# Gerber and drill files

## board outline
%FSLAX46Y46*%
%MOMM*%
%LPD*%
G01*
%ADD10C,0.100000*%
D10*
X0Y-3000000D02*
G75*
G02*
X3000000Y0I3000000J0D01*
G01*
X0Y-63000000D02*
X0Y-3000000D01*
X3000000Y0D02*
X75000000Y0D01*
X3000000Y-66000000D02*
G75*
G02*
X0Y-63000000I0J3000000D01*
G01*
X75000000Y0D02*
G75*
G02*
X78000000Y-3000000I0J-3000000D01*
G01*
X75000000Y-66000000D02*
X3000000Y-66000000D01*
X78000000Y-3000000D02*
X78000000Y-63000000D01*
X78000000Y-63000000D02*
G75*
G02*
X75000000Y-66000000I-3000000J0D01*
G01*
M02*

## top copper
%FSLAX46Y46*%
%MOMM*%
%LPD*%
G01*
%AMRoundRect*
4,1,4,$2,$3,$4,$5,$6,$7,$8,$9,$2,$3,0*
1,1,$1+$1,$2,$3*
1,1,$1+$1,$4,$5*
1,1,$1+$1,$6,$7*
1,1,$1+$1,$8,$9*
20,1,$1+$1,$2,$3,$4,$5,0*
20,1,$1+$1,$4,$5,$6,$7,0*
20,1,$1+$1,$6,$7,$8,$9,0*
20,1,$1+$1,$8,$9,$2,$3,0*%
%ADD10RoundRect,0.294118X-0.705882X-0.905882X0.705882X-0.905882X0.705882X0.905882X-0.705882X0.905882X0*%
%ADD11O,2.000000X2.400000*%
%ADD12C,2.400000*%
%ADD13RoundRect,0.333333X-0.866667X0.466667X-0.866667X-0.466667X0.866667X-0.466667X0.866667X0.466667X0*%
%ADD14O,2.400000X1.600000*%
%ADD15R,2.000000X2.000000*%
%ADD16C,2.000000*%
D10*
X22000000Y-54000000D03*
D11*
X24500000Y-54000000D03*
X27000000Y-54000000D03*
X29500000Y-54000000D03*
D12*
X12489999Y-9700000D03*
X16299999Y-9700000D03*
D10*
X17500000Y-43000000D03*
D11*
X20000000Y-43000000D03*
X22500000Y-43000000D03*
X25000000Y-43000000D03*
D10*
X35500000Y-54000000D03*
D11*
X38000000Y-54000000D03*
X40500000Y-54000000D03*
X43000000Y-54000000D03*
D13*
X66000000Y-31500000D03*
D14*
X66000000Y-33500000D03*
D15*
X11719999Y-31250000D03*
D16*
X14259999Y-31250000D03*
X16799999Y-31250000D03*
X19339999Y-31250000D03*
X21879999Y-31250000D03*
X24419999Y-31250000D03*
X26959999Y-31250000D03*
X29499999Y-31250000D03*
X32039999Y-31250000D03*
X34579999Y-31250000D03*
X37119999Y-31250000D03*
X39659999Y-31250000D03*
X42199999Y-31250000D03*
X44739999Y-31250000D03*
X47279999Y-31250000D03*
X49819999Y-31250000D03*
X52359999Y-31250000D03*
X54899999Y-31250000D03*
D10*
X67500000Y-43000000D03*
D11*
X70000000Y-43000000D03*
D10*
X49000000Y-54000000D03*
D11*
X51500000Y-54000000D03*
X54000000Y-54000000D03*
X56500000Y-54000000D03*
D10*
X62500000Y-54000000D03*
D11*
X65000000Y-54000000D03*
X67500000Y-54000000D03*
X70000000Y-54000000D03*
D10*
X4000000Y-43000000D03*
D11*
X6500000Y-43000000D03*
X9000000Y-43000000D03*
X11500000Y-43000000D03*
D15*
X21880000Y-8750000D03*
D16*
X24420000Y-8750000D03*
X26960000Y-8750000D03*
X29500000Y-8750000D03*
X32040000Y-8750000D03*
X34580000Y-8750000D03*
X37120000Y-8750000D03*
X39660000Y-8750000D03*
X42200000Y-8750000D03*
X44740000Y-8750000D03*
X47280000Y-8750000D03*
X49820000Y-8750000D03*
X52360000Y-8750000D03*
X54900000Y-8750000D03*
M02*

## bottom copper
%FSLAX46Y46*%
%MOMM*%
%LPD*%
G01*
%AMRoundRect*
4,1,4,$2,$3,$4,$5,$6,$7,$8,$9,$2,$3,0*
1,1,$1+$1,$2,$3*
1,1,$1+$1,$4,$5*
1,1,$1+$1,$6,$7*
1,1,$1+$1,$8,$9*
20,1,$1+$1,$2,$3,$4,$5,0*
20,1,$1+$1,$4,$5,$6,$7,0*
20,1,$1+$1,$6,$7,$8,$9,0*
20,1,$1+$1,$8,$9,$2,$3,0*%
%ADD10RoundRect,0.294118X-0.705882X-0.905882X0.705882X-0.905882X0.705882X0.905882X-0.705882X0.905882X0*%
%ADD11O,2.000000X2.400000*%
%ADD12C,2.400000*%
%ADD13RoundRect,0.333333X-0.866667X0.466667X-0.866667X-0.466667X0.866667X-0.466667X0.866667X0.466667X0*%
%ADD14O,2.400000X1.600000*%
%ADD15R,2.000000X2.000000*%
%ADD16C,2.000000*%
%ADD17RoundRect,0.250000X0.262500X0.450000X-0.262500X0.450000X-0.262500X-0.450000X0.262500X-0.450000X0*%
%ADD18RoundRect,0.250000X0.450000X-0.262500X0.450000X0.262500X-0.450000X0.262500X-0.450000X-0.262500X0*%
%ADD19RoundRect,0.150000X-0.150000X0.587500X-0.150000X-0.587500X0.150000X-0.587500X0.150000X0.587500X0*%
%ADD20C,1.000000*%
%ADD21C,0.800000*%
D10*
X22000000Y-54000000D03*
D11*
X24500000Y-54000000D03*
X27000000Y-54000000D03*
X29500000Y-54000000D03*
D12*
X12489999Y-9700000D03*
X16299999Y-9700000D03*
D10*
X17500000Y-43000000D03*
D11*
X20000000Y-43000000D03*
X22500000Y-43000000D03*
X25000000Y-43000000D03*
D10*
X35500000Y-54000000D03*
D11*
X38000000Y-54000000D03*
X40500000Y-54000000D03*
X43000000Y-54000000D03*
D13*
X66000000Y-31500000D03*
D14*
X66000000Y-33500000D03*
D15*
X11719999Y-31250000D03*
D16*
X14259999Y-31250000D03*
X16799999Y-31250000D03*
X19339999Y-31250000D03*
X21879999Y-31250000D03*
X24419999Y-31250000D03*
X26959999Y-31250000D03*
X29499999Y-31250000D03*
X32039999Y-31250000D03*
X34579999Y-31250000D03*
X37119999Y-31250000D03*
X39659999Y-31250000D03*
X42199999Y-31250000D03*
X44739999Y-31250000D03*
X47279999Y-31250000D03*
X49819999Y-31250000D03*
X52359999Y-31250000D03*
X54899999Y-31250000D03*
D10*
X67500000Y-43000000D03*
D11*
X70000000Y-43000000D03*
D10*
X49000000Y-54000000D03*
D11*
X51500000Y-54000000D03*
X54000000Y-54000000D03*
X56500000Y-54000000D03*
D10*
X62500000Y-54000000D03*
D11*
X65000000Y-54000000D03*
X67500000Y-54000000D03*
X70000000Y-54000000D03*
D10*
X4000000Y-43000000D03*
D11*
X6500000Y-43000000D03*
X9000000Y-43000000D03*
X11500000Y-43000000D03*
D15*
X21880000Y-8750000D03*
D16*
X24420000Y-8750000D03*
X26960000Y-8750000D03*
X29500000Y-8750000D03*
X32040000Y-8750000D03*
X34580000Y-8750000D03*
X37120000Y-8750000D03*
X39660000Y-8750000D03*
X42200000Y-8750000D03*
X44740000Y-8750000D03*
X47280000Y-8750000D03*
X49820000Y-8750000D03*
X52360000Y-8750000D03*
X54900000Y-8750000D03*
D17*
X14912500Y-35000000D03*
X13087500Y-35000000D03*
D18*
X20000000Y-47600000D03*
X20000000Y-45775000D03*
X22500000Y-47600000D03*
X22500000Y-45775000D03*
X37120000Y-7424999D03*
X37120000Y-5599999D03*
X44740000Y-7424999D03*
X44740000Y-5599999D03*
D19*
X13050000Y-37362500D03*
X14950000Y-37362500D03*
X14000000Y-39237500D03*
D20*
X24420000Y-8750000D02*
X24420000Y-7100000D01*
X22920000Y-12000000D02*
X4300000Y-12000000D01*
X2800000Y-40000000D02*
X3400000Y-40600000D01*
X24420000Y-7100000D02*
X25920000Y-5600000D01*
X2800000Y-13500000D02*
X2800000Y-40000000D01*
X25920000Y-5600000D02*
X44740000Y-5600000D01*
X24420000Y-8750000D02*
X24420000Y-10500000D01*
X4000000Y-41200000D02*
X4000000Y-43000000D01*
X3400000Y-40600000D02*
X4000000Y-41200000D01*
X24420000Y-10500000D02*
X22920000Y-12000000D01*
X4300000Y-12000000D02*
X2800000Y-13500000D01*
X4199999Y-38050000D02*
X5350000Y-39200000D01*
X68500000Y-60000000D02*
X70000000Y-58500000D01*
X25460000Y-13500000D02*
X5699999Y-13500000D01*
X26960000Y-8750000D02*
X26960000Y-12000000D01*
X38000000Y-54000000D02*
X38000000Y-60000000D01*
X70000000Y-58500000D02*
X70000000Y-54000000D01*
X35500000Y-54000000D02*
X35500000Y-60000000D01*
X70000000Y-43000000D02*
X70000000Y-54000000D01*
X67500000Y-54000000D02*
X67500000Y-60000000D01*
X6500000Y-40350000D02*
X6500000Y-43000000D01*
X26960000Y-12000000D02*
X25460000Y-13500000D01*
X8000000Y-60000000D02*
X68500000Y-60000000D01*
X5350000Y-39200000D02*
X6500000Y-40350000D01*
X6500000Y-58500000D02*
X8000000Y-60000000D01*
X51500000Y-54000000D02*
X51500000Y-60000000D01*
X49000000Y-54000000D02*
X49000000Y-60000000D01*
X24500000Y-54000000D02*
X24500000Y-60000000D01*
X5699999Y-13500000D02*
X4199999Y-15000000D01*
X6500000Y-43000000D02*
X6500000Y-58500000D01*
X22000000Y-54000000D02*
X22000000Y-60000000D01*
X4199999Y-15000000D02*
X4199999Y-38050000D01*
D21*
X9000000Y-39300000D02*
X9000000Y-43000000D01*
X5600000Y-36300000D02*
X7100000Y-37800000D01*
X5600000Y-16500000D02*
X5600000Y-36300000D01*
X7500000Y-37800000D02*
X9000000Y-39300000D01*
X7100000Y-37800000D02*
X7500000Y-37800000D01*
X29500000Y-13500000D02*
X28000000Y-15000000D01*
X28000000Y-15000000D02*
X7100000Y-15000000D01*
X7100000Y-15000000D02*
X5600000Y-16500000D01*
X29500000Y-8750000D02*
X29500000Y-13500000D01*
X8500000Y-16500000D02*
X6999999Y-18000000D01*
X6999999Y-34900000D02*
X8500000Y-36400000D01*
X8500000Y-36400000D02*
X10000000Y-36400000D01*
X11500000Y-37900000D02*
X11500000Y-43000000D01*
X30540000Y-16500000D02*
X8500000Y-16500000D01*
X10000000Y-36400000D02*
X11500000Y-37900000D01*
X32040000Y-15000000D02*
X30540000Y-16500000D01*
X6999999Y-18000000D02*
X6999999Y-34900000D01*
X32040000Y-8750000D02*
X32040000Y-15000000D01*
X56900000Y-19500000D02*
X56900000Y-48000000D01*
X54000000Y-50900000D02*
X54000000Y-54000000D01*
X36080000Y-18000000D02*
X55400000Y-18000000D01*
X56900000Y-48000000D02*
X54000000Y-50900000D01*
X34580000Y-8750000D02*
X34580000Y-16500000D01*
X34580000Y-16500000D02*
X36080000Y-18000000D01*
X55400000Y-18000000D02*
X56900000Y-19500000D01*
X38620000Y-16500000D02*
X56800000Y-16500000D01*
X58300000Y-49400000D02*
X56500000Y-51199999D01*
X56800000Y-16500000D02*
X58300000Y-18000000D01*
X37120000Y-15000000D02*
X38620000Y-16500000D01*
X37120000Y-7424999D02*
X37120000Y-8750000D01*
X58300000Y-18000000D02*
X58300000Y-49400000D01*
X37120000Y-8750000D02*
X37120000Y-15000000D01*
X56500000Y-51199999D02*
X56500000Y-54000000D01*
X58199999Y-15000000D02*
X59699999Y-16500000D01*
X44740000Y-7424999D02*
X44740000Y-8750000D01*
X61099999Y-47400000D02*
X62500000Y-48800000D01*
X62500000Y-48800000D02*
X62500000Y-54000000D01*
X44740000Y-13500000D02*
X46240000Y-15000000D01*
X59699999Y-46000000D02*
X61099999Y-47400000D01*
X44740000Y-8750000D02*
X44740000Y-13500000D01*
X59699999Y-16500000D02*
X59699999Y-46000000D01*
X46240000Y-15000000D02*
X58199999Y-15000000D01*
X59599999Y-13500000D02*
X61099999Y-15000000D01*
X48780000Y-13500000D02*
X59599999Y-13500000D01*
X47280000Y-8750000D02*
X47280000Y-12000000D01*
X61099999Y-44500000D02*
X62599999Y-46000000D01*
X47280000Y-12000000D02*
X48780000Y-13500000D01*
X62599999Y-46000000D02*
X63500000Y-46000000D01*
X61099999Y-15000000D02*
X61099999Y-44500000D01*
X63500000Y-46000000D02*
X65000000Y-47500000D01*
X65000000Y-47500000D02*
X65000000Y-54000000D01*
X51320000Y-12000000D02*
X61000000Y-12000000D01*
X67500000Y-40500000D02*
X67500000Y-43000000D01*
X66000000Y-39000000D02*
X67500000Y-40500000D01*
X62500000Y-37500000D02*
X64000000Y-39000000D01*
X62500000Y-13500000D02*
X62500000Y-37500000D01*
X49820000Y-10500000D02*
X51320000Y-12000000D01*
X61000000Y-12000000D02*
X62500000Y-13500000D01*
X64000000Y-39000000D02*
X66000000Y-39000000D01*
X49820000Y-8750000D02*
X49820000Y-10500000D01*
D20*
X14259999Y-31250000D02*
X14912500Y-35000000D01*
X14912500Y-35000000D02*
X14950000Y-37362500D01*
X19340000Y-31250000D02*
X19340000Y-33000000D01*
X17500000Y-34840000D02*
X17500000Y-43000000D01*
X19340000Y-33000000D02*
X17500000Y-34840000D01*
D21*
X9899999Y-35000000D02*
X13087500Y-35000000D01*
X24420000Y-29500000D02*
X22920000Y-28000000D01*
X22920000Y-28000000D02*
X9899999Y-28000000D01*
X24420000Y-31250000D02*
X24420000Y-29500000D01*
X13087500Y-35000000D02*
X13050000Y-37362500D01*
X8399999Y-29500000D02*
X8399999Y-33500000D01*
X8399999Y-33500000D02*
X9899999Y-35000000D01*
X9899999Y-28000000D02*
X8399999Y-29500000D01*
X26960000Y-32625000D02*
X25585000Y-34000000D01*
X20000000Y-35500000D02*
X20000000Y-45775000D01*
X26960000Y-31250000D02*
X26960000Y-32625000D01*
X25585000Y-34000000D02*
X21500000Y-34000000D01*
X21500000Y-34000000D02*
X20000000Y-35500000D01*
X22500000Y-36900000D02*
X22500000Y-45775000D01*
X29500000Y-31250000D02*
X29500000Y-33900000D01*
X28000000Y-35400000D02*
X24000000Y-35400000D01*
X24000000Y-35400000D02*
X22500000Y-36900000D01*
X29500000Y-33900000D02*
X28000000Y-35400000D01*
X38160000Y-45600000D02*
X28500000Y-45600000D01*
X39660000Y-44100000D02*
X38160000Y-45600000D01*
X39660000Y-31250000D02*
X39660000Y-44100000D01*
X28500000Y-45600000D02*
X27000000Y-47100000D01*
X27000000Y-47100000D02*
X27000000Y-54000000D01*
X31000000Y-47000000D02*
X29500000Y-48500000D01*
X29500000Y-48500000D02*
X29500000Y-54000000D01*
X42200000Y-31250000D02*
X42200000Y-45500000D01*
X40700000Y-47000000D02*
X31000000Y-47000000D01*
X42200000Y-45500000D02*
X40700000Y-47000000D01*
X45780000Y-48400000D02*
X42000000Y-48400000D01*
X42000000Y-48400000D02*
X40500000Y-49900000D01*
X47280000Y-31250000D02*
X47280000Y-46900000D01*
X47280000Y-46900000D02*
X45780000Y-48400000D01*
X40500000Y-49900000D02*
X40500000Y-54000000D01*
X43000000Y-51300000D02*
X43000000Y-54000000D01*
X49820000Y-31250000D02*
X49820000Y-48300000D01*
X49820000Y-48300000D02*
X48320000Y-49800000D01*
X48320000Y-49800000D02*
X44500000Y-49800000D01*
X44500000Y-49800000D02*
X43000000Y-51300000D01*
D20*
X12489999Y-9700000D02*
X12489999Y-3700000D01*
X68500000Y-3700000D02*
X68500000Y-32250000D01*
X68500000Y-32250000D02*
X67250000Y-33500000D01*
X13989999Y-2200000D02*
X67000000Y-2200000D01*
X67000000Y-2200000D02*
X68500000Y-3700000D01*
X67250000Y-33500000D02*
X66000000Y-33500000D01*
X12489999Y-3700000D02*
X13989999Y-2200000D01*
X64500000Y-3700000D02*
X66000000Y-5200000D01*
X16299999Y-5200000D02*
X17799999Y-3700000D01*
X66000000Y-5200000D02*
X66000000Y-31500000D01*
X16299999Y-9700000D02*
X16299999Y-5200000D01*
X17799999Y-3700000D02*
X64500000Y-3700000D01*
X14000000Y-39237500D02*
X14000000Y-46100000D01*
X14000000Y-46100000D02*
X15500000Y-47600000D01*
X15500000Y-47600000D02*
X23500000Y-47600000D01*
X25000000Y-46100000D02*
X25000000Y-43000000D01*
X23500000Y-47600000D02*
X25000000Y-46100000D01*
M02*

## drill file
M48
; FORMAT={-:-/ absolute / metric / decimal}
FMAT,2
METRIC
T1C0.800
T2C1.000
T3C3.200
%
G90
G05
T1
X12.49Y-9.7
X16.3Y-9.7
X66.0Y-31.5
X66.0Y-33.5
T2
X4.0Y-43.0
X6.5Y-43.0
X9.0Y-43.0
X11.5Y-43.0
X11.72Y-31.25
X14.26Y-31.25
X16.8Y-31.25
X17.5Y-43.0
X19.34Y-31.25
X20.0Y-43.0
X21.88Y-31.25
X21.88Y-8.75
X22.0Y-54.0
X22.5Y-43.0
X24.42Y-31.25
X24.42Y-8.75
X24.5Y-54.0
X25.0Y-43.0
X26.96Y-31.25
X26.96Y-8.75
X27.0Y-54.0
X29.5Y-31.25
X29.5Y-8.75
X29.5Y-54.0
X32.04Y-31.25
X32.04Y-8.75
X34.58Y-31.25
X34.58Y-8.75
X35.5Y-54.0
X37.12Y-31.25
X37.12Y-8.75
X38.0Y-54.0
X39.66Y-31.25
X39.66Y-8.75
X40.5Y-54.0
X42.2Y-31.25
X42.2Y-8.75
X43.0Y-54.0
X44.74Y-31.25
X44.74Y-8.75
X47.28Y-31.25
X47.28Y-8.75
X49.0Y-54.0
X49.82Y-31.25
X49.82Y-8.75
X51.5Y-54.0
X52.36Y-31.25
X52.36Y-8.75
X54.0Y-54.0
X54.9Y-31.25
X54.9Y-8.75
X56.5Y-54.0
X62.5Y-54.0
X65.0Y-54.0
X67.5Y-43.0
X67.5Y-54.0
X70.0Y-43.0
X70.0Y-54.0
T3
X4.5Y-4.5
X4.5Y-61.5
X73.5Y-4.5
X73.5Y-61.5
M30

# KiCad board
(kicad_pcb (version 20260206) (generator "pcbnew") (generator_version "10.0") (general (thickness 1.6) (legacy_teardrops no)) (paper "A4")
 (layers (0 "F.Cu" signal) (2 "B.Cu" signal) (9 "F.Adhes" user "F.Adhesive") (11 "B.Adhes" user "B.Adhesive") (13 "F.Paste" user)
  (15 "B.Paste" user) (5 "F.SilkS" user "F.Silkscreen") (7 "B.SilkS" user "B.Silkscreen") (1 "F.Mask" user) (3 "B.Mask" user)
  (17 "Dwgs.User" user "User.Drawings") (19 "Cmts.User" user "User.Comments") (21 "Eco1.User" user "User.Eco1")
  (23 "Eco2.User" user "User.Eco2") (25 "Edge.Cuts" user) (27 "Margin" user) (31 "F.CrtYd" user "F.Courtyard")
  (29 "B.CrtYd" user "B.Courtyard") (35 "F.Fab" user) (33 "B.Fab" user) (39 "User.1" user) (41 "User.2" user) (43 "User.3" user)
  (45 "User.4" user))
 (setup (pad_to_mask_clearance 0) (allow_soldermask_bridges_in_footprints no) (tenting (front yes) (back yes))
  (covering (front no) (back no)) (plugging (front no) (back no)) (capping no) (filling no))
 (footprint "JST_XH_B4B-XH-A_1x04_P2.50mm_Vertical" (layer "F.Cu") (at 22 54)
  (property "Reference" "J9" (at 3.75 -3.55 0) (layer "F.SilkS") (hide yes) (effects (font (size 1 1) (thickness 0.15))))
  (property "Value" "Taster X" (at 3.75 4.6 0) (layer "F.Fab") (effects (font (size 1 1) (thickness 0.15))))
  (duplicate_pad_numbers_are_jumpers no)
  (pad "1" thru_hole roundrect (at 0 0) (size 2 2.4) (drill 1) (layers "*.Cu" "*.Mask") (remove_unused_layers no)
   (roundrect_rratio 0.147059) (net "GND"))
  (pad "2" thru_hole oval (at 2.5 0) (size 2 2.4) (drill 1) (layers "*.Cu" "*.Mask") (remove_unused_layers no) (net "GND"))
  (pad "3" thru_hole oval (at 5 0) (size 2 2.4) (drill 1) (layers "*.Cu" "*.Mask") (remove_unused_layers no) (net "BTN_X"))
  (pad "4" thru_hole oval (at 7.5 0) (size 2 2.4) (drill 1) (layers "*.Cu" "*.Mask") (remove_unused_layers no) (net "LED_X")))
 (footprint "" (layer "F.Cu") (at 12.489999 9.7)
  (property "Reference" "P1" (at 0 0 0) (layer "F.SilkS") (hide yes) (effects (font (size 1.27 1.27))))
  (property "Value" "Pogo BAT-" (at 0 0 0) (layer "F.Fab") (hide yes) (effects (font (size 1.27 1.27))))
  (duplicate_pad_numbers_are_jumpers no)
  (pad "1" thru_hole circle (at 0 0) (size 2.4 2.4) (drill 0.8) (layers "*.Cu" "*.Mask") (remove_unused_layers no) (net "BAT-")))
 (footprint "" (layer "F.Cu") (at 16.299999 9.7)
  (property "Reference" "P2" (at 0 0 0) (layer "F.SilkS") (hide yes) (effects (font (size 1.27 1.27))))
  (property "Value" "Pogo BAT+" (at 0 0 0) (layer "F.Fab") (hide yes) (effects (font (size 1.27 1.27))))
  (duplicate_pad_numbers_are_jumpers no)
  (pad "1" thru_hole circle (at 0 0) (size 2.4 2.4) (drill 0.8) (layers "*.Cu" "*.Mask") (remove_unused_layers no) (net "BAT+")))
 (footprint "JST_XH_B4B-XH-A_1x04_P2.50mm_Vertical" (layer "F.Cu") (at 17.5 43)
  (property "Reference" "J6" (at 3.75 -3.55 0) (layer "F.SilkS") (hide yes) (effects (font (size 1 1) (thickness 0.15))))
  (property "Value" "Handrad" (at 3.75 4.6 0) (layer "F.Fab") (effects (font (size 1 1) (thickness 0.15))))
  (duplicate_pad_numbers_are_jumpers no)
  (pad "1" thru_hole roundrect (at 0 0) (size 2 2.4) (drill 1) (layers "*.Cu" "*.Mask") (remove_unused_layers no)
   (roundrect_rratio 0.147059) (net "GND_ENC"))
  (pad "2" thru_hole oval (at 2.5 0) (size 2 2.4) (drill 1) (layers "*.Cu" "*.Mask") (remove_unused_layers no) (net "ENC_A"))
  (pad "3" thru_hole oval (at 5 0) (size 2 2.4) (drill 1) (layers "*.Cu" "*.Mask") (remove_unused_layers no) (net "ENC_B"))
  (pad "4" thru_hole oval (at 7.5 0) (size 2 2.4) (drill 1) (layers "*.Cu" "*.Mask") (remove_unused_layers no) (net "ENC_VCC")))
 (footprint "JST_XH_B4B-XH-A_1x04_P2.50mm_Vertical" (layer "F.Cu") (at 35.5 54)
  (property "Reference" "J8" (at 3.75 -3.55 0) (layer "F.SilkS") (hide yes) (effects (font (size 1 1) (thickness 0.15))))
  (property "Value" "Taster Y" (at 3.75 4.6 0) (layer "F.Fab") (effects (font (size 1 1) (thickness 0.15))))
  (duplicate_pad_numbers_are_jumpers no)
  (pad "1" thru_hole roundrect (at 0 0) (size 2 2.4) (drill 1) (layers "*.Cu" "*.Mask") (remove_unused_layers no)
   (roundrect_rratio 0.147059) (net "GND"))
  (pad "2" thru_hole oval (at 2.5 0) (size 2 2.4) (drill 1) (layers "*.Cu" "*.Mask") (remove_unused_layers no) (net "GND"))
  (pad "3" thru_hole oval (at 5 0) (size 2 2.4) (drill 1) (layers "*.Cu" "*.Mask") (remove_unused_layers no) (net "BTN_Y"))
  (pad "4" thru_hole oval (at 7.5 0) (size 2 2.4) (drill 1) (layers "*.Cu" "*.Mask") (remove_unused_layers no) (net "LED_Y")))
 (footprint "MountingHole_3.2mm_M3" (layer "F.Cu") (at 4.5 61.5)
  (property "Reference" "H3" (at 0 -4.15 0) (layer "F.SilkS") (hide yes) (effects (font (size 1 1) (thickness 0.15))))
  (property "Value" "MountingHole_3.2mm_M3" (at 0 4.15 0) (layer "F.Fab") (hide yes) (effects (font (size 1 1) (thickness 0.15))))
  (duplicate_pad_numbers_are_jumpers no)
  (pad "" np_thru_hole circle (at 0 0) (size 3.2 3.2) (drill 3.2) (layers "*.Cu" "*.Mask")))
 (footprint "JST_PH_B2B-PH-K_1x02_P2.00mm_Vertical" (layer "F.Cu") (at 66 31.5 -90)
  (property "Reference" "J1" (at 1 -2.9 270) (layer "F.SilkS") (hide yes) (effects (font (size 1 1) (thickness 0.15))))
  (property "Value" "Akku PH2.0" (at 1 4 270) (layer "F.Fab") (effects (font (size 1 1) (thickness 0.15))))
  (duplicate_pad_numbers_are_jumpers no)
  (pad "1" thru_hole roundrect (at 0 0 270) (size 1.6 2.4) (drill 0.8) (layers "*.Cu" "*.Mask") (remove_unused_layers no)
   (roundrect_rratio 0.208333) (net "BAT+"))
  (pad "2" thru_hole oval (at 2 0 270) (size 1.6 2.4) (drill 0.8) (layers "*.Cu" "*.Mask") (remove_unused_layers no) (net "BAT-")))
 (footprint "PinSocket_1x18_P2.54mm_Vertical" (layer "F.Cu") (at 11.719999 31.25 90)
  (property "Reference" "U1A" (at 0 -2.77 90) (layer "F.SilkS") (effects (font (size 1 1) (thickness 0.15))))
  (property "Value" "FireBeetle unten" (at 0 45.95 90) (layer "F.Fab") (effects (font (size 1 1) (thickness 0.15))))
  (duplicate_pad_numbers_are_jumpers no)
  (pad "1" thru_hole rect (at 0 0 90) (size 2 2) (drill 1) (layers "*.Cu" "*.Mask") (remove_unused_layers no))
  (pad "2" thru_hole circle (at 0 2.54 90) (size 2 2) (drill 1) (layers "*.Cu" "*.Mask") (remove_unused_layers no) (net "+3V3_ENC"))
  (pad "3" thru_hole circle (at 0 5.08 90) (size 2 2) (drill 1) (layers "*.Cu" "*.Mask") (remove_unused_layers no))
  (pad "4" thru_hole circle (at 0 7.62 90) (size 2 2) (drill 1) (layers "*.Cu" "*.Mask") (remove_unused_layers no) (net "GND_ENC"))
  (pad "5" thru_hole circle (at 0 10.16 90) (size 2 2) (drill 1) (layers "*.Cu" "*.Mask") (remove_unused_layers no))
  (pad "6" thru_hole circle (at 0 12.7 90) (size 2 2) (drill 1) (layers "*.Cu" "*.Mask") (remove_unused_layers no) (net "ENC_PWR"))
  (pad "7" thru_hole circle (at 0 15.24 90) (size 2 2) (drill 1) (layers "*.Cu" "*.Mask") (remove_unused_layers no) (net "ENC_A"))
  (pad "8" thru_hole circle (at 0 17.78 90) (size 2 2) (drill 1) (layers "*.Cu" "*.Mask") (remove_unused_layers no) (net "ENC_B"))
  (pad "9" thru_hole circle (at 0 20.32 90) (size 2 2) (drill 1) (layers "*.Cu" "*.Mask") (remove_unused_layers no))
  (pad "10" thru_hole circle (at 0 22.86 90) (size 2 2) (drill 1) (layers "*.Cu" "*.Mask") (remove_unused_layers no))
  (pad "11" thru_hole circle (at 0 25.4 90) (size 2 2) (drill 1) (layers "*.Cu" "*.Mask") (remove_unused_layers no))
  (pad "12" thru_hole circle (at 0 27.94 90) (size 2 2) (drill 1) (layers "*.Cu" "*.Mask") (remove_unused_layers no) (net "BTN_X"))
  (pad "13" thru_hole circle (at 0 30.48 90) (size 2 2) (drill 1) (layers "*.Cu" "*.Mask") (remove_unused_layers no) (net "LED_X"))
  (pad "14" thru_hole circle (at 0 33.02 90) (size 2 2) (drill 1) (layers "*.Cu" "*.Mask") (remove_unused_layers no))
  (pad "15" thru_hole circle (at 0 35.56 90) (size 2 2) (drill 1) (layers "*.Cu" "*.Mask") (remove_unused_layers no) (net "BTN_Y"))
  (pad "16" thru_hole circle (at 0 38.1 90) (size 2 2) (drill 1) (layers "*.Cu" "*.Mask") (remove_unused_layers no) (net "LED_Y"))
  (pad "17" thru_hole circle (at 0 40.64 90) (size 2 2) (drill 1) (layers "*.Cu" "*.Mask") (remove_unused_layers no))
  (pad "18" thru_hole circle (at 0 43.18 90) (size 2 2) (drill 1) (layers "*.Cu" "*.Mask") (remove_unused_layers no)))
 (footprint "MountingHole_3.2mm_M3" (layer "F.Cu") (at 73.5 4.5)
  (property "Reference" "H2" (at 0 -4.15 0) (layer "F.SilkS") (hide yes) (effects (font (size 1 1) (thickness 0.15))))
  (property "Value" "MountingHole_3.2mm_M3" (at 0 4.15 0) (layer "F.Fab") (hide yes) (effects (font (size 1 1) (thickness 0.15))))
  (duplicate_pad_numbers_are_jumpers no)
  (pad "" np_thru_hole circle (at 0 0) (size 3.2 3.2) (drill 3.2) (layers "*.Cu" "*.Mask")))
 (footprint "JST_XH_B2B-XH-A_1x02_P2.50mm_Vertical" (layer "F.Cu") (at 67.5 43)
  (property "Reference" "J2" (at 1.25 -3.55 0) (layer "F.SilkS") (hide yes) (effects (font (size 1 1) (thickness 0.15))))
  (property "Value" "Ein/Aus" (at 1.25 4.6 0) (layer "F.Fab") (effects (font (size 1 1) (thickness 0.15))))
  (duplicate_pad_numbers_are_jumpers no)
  (pad "1" thru_hole roundrect (at 0 0) (size 2 2.4) (drill 1) (layers "*.Cu" "*.Mask") (remove_unused_layers no)
   (roundrect_rratio 0.147059) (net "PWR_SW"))
  (pad "2" thru_hole oval (at 2.5 0) (size 2 2.4) (drill 1) (layers "*.Cu" "*.Mask") (remove_unused_layers no) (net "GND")))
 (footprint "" (layer "F.Cu") (at 30.4 20 90)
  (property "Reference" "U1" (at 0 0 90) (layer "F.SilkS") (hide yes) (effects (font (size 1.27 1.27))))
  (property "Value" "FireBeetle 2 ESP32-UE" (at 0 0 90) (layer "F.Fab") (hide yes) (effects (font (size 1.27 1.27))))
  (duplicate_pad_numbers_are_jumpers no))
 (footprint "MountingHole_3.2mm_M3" (layer "F.Cu") (at 73.5 61.5)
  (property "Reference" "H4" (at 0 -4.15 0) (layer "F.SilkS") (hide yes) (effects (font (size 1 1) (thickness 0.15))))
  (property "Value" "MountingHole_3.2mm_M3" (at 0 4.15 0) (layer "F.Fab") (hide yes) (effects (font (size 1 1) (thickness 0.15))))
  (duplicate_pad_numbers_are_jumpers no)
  (pad "" np_thru_hole circle (at 0 0) (size 3.2 3.2) (drill 3.2) (layers "*.Cu" "*.Mask")))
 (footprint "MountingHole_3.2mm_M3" (layer "F.Cu") (at 4.5 4.5)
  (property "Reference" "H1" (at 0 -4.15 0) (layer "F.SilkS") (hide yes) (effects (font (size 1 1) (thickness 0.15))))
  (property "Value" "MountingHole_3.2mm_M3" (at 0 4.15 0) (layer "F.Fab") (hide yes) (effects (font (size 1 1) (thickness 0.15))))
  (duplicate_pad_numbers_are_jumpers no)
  (pad "" np_thru_hole circle (at 0 0) (size 3.2 3.2) (drill 3.2) (layers "*.Cu" "*.Mask")))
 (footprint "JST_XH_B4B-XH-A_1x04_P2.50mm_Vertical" (layer "F.Cu") (at 49 54)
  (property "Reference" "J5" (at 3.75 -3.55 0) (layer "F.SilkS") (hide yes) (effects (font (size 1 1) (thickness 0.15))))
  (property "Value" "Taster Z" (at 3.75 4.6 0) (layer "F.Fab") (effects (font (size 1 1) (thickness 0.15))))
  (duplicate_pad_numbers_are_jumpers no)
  (pad "1" thru_hole roundrect (at 0 0) (size 2 2.4) (drill 1) (layers "*.Cu" "*.Mask") (remove_unused_layers no)
   (roundrect_rratio 0.147059) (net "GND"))
  (pad "2" thru_hole oval (at 2.5 0) (size 2 2.4) (drill 1) (layers "*.Cu" "*.Mask") (remove_unused_layers no) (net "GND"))
  (pad "3" thru_hole oval (at 5 0) (size 2 2.4) (drill 1) (layers "*.Cu" "*.Mask") (remove_unused_layers no) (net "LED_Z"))
  (pad "4" thru_hole oval (at 7.5 0) (size 2 2.4) (drill 1) (layers "*.Cu" "*.Mask") (remove_unused_layers no) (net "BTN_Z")))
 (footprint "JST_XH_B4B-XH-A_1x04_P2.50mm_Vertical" (layer "F.Cu") (at 62.5 54)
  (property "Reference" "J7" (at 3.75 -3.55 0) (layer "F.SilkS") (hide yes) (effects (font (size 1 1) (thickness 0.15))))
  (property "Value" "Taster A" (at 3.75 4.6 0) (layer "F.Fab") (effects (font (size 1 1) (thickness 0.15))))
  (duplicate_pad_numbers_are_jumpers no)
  (pad "1" thru_hole roundrect (at 0 0) (size 2 2.4) (drill 1) (layers "*.Cu" "*.Mask") (remove_unused_layers no)
   (roundrect_rratio 0.147059) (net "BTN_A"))
  (pad "2" thru_hole oval (at 2.5 0) (size 2 2.4) (drill 1) (layers "*.Cu" "*.Mask") (remove_unused_layers no) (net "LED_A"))
  (pad "3" thru_hole oval (at 5 0) (size 2 2.4) (drill 1) (layers "*.Cu" "*.Mask") (remove_unused_layers no) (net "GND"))
  (pad "4" thru_hole oval (at 7.5 0) (size 2 2.4) (drill 1) (layers "*.Cu" "*.Mask") (remove_unused_layers no) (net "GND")))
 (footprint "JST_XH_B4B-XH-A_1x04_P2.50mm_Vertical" (layer "F.Cu") (at 4 43)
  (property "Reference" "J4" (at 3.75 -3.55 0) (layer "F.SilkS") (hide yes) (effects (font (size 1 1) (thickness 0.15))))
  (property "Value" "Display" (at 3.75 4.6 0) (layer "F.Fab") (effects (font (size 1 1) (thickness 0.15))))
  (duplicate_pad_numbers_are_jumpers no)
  (pad "1" thru_hole roundrect (at 0 0) (size 2 2.4) (drill 1) (layers "*.Cu" "*.Mask") (remove_unused_layers no)
   (roundrect_rratio 0.147059) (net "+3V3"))
  (pad "2" thru_hole oval (at 2.5 0) (size 2 2.4) (drill 1) (layers "*.Cu" "*.Mask") (remove_unused_layers no) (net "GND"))
  (pad "3" thru_hole oval (at 5 0) (size 2 2.4) (drill 1) (layers "*.Cu" "*.Mask") (remove_unused_layers no) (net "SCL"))
  (pad "4" thru_hole oval (at 7.5 0) (size 2 2.4) (drill 1) (layers "*.Cu" "*.Mask") (remove_unused_layers no) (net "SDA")))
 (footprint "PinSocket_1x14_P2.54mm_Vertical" (layer "F.Cu") (at 21.88 8.75 90)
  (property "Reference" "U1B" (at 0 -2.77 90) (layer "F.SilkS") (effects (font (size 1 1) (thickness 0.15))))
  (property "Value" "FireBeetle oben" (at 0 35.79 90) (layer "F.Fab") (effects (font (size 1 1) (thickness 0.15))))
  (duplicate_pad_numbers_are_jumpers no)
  (pad "1" thru_hole rect (at 0 0 90) (size 2 2) (drill 1) (layers "*.Cu" "*.Mask") (remove_unused_layers no))
  (pad "2" thru_hole circle (at 0 2.54 90) (size 2 2) (drill 1) (layers "*.Cu" "*.Mask") (remove_unused_layers no) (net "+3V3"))
  (pad "3" thru_hole circle (at 0 5.08 90) (size 2 2) (drill 1) (layers "*.Cu" "*.Mask") (remove_unused_layers no) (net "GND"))
  (pad "4" thru_hole circle (at 0 7.62 90) (size 2 2) (drill 1) (layers "*.Cu" "*.Mask") (remove_unused_layers no) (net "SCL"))
  (pad "5" thru_hole circle (at 0 10.16 90) (size 2 2) (drill 1) (layers "*.Cu" "*.Mask") (remove_unused_layers no) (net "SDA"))
  (pad "6" thru_hole circle (at 0 12.7 90) (size 2 2) (drill 1) (layers "*.Cu" "*.Mask") (remove_unused_layers no) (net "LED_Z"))
  (pad "7" thru_hole circle (at 0 15.24 90) (size 2 2) (drill 1) (layers "*.Cu" "*.Mask") (remove_unused_layers no) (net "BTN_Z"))
  (pad "8" thru_hole circle (at 0 17.78 90) (size 2 2) (drill 1) (layers "*.Cu" "*.Mask") (remove_unused_layers no))
  (pad "9" thru_hole circle (at 0 20.32 90) (size 2 2) (drill 1) (layers "*.Cu" "*.Mask") (remove_unused_layers no))
  (pad "10" thru_hole circle (at 0 22.86 90) (size 2 2) (drill 1) (layers "*.Cu" "*.Mask") (remove_unused_layers no) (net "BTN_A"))
  (pad "11" thru_hole circle (at 0 25.4 90) (size 2 2) (drill 1) (layers "*.Cu" "*.Mask") (remove_unused_layers no) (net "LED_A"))
  (pad "12" thru_hole circle (at 0 27.94 90) (size 2 2) (drill 1) (layers "*.Cu" "*.Mask") (remove_unused_layers no) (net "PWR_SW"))
  (pad "13" thru_hole circle (at 0 30.48 90) (size 2 2) (drill 1) (layers "*.Cu" "*.Mask") (remove_unused_layers no))
  (pad "14" thru_hole circle (at 0 33.02 90) (size 2 2) (drill 1) (layers "*.Cu" "*.Mask") (remove_unused_layers no)))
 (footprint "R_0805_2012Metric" (layer "B.Cu") (at 14 35 180)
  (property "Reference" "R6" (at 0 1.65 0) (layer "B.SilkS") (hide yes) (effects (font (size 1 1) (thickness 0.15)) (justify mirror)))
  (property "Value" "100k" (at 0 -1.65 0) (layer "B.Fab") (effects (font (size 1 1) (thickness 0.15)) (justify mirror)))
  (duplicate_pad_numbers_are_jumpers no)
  (pad "1" smd roundrect (at -0.9125 0 180) (size 1.025 1.4) (layers "B.Cu" "B.Mask" "B.Paste") (roundrect_rratio 0.243902) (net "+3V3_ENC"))
  (pad "2" smd roundrect (at 0.9125 0 180) (size 1.025 1.4) (layers "B.Cu" "B.Mask" "B.Paste") (roundrect_rratio 0.243902) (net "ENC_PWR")))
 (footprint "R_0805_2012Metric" (layer "B.Cu") (at 20 46.6875 90)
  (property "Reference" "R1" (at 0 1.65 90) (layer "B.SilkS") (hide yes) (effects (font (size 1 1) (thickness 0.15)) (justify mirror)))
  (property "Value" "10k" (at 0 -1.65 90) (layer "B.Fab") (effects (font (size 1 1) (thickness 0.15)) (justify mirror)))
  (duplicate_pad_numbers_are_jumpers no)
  (pad "1" smd roundrect (at -0.9125 0 90) (size 1.025 1.4) (layers "B.Cu" "B.Mask" "B.Paste") (roundrect_rratio 0.243902) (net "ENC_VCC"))
  (pad "2" smd roundrect (at 0.9125 0 90) (size 1.025 1.4) (layers "B.Cu" "B.Mask" "B.Paste") (roundrect_rratio 0.243902) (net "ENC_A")))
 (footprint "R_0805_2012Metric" (layer "B.Cu") (at 22.5 46.6875 90)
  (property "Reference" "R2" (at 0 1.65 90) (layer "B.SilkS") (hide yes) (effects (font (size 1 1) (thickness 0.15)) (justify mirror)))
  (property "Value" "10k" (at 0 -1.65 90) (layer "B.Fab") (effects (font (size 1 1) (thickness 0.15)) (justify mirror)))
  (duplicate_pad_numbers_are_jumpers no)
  (pad "1" smd roundrect (at -0.9125 0 90) (size 1.025 1.4) (layers "B.Cu" "B.Mask" "B.Paste") (roundrect_rratio 0.243902) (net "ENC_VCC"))
  (pad "2" smd roundrect (at 0.9125 0 90) (size 1.025 1.4) (layers "B.Cu" "B.Mask" "B.Paste") (roundrect_rratio 0.243902) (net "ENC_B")))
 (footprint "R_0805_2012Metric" (layer "B.Cu") (at 37.12 6.512499 90)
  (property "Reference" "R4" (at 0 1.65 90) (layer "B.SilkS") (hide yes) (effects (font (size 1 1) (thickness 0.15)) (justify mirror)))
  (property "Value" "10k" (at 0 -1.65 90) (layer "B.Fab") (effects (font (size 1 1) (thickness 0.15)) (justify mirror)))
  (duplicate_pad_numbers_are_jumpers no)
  (pad "1" smd roundrect (at -0.9125 0 90) (size 1.025 1.4) (layers "B.Cu" "B.Mask" "B.Paste") (roundrect_rratio 0.243902) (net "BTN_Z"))
  (pad "2" smd roundrect (at 0.9125 0 90) (size 1.025 1.4) (layers "B.Cu" "B.Mask" "B.Paste") (roundrect_rratio 0.243902) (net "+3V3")))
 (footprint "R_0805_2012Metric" (layer "B.Cu") (at 44.74 6.512499 90)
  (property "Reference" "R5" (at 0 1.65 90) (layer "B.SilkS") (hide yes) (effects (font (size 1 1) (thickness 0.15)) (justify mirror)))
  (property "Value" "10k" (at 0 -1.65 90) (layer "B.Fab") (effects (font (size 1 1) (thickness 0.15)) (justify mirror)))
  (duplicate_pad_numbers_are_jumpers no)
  (pad "1" smd roundrect (at -0.9125 0 90) (size 1.025 1.4) (layers "B.Cu" "B.Mask" "B.Paste") (roundrect_rratio 0.243902) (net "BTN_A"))
  (pad "2" smd roundrect (at 0.9125 0 90) (size 1.025 1.4) (layers "B.Cu" "B.Mask" "B.Paste") (roundrect_rratio 0.243902) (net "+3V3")))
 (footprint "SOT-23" (layer "B.Cu") (at 14 38.3 -90)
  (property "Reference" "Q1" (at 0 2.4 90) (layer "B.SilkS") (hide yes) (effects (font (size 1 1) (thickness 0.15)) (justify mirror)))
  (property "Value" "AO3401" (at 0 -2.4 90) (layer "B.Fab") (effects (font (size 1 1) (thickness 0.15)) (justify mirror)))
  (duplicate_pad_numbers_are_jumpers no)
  (pad "1" smd roundrect (at -0.9375 0.95 270) (size 1.475 0.6) (layers "B.Cu" "B.Mask" "B.Paste") (roundrect_rratio 0.25) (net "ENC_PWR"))
  (pad "2" smd roundrect (at -0.9375 -0.95 270) (size 1.475 0.6) (layers "B.Cu" "B.Mask" "B.Paste") (roundrect_rratio 0.25) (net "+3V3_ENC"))
  (pad "3" smd roundrect (at 0.9375 0 270) (size 1.475 0.6) (layers "B.Cu" "B.Mask" "B.Paste") (roundrect_rratio 0.25) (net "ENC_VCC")))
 (gr_arc (start 0 3) (mid 0.87868 0.87868) (end 3 0) (stroke (width 0.1) (type default)) (layer "Edge.Cuts"))
 (gr_line (start 0 63) (end 0 3) (stroke (width 0.1) (type default)) (layer "Edge.Cuts"))
 (gr_line (start 3 0) (end 75 0) (stroke (width 0.1) (type default)) (layer "Edge.Cuts"))
 (gr_arc (start 3 66) (mid 0.87868 65.12132) (end 0 63) (stroke (width 0.1) (type default)) (layer "Edge.Cuts"))
 (gr_arc (start 75 0) (mid 77.12132 0.87868) (end 78 3) (stroke (width 0.1) (type default)) (layer "Edge.Cuts"))
 (gr_line (start 75 66) (end 3 66) (stroke (width 0.1) (type default)) (layer "Edge.Cuts"))
 (gr_line (start 78 3) (end 78 63) (stroke (width 0.1) (type default)) (layer "Edge.Cuts"))
 (gr_arc (start 78 63) (mid 77.12132 65.12132) (end 75 66) (stroke (width 0.1) (type default)) (layer "Edge.Cuts"))
 (segment (start 24.42 8.75) (end 24.42 7.1) (width 1) (layer "B.Cu") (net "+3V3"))
 (segment (start 22.92 12) (end 4.3 12) (width 1) (layer "B.Cu") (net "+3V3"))
 (segment (start 2.8 40) (end 3.4 40.6) (width 1) (layer "B.Cu") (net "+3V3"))
 (segment (start 24.42 7.1) (end 25.92 5.6) (width 1) (layer "B.Cu") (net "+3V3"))
 (segment (start 2.8 13.5) (end 2.8 40) (width 1) (layer "B.Cu") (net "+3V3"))
 (segment (start 25.92 5.6) (end 44.74 5.6) (width 1) (layer "B.Cu") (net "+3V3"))
 (segment (start 24.42 8.75) (end 24.42 10.5) (width 1) (layer "B.Cu") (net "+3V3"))
 (segment (start 4 41.2) (end 4 43) (width 1) (layer "B.Cu") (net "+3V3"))
 (segment (start 3.4 40.6) (end 4 41.2) (width 1) (layer "B.Cu") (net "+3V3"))
 (segment (start 24.42 10.5) (end 22.92 12) (width 1) (layer "B.Cu") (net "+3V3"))
 (segment (start 4.3 12) (end 2.8 13.5) (width 1) (layer "B.Cu") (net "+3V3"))
 (segment (start 4.199999 38.05) (end 5.35 39.2) (width 1) (layer "B.Cu") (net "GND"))
 (segment (start 68.5 60) (end 70 58.5) (width 1) (layer "B.Cu") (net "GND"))
 (segment (start 25.46 13.5) (end 5.699999 13.5) (width 1) (layer "B.Cu") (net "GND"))
 (segment (start 26.96 8.75) (end 26.96 12) (width 1) (layer "B.Cu") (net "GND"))
 (segment (start 38 54) (end 38 60) (width 1) (layer "B.Cu") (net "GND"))
 (segment (start 70 58.5) (end 70 54) (width 1) (layer "B.Cu") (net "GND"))
 (segment (start 35.5 54) (end 35.5 60) (width 1) (layer "B.Cu") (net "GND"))
 (segment (start 70 43) (end 70 54) (width 1) (layer "B.Cu") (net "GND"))
 (segment (start 67.5 54) (end 67.5 60) (width 1) (layer "B.Cu") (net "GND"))
 (segment (start 6.5 40.35) (end 6.5 43) (width 1) (layer "B.Cu") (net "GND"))
 (segment (start 26.96 12) (end 25.46 13.5) (width 1) (layer "B.Cu") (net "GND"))
 (segment (start 8 60) (end 68.5 60) (width 1) (layer "B.Cu") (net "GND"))
 (segment (start 5.35 39.2) (end 6.5 40.35) (width 1) (layer "B.Cu") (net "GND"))
 (segment (start 6.5 58.5) (end 8 60) (width 1) (layer "B.Cu") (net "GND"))
 (segment (start 51.5 54) (end 51.5 60) (width 1) (layer "B.Cu") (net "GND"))
 (segment (start 49 54) (end 49 60) (width 1) (layer "B.Cu") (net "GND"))
 (segment (start 24.5 54) (end 24.5 60) (width 1) (layer "B.Cu") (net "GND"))
 (segment (start 5.699999 13.5) (end 4.199999 15) (width 1) (layer "B.Cu") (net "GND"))
 (segment (start 6.5 43) (end 6.5 58.5) (width 1) (layer "B.Cu") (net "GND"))
 (segment (start 22 54) (end 22 60) (width 1) (layer "B.Cu") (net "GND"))
 (segment (start 4.199999 15) (end 4.199999 38.05) (width 1) (layer "B.Cu") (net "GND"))
 (segment (start 9 39.3) (end 9 43) (width 0.8) (layer "B.Cu") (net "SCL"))
 (segment (start 5.6 36.3) (end 7.1 37.8) (width 0.8) (layer "B.Cu") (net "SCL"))
 (segment (start 5.6 16.5) (end 5.6 36.3) (width 0.8) (layer "B.Cu") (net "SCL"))
 (segment (start 7.5 37.8) (end 9 39.3) (width 0.8) (layer "B.Cu") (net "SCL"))
 (segment (start 7.1 37.8) (end 7.5 37.8) (width 0.8) (layer "B.Cu") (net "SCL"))
 (segment (start 29.5 13.5) (end 28 15) (width 0.8) (layer "B.Cu") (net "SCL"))
 (segment (start 28 15) (end 7.1 15) (width 0.8) (layer "B.Cu") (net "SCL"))
 (segment (start 7.1 15) (end 5.6 16.5) (width 0.8) (layer "B.Cu") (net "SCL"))
 (segment (start 29.5 8.75) (end 29.5 13.5) (width 0.8) (layer "B.Cu") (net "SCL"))
 (segment (start 8.5 16.5) (end 6.999999 18) (width 0.8) (layer "B.Cu") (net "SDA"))
 (segment (start 6.999999 34.9) (end 8.5 36.4) (width 0.8) (layer "B.Cu") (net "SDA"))
 (segment (start 8.5 36.4) (end 10 36.4) (width 0.8) (layer "B.Cu") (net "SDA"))
 (segment (start 11.5 37.9) (end 11.5 43) (width 0.8) (layer "B.Cu") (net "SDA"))
 (segment (start 30.54 16.5) (end 8.5 16.5) (width 0.8) (layer "B.Cu") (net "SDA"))
 (segment (start 10 36.4) (end 11.5 37.9) (width 0.8) (layer "B.Cu") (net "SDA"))
 (segment (start 32.04 15) (end 30.54 16.5) (width 0.8) (layer "B.Cu") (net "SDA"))
 (segment (start 6.999999 18) (end 6.999999 34.9) (width 0.8) (layer "B.Cu") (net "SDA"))
 (segment (start 32.04 8.75) (end 32.04 15) (width 0.8) (layer "B.Cu") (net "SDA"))
 (segment (start 56.9 19.5) (end 56.9 48) (width 0.8) (layer "B.Cu") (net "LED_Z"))
 (segment (start 54 50.9) (end 54 54) (width 0.8) (layer "B.Cu") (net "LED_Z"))
 (segment (start 36.08 18) (end 55.4 18) (width 0.8) (layer "B.Cu") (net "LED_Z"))
 (segment (start 56.9 48) (end 54 50.9) (width 0.8) (layer "B.Cu") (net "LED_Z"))
 (segment (start 34.58 8.75) (end 34.58 16.5) (width 0.8) (layer "B.Cu") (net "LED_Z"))
 (segment (start 34.58 16.5) (end 36.08 18) (width 0.8) (layer "B.Cu") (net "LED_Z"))
 (segment (start 55.4 18) (end 56.9 19.5) (width 0.8) (layer "B.Cu") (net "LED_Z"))
 (segment (start 38.62 16.5) (end 56.8 16.5) (width 0.8) (layer "B.Cu") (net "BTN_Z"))
 (segment (start 58.3 49.4) (end 56.5 51.199999) (width 0.8) (layer "B.Cu") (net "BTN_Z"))
 (segment (start 56.8 16.5) (end 58.3 18) (width 0.8) (layer "B.Cu") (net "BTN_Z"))
 (segment (start 37.12 15) (end 38.62 16.5) (width 0.8) (layer "B.Cu") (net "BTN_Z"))
 (segment (start 37.12 7.424999) (end 37.12 8.75) (width 0.8) (layer "B.Cu") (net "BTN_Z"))
 (segment (start 58.3 18) (end 58.3 49.4) (width 0.8) (layer "B.Cu") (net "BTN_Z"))
 (segment (start 37.12 8.75) (end 37.12 15) (width 0.8) (layer "B.Cu") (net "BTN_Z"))
 (segment (start 56.5 51.199999) (end 56.5 54) (width 0.8) (layer "B.Cu") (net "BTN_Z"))
 (segment (start 58.199999 15) (end 59.699999 16.5) (width 0.8) (layer "B.Cu") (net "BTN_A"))
 (segment (start 44.74 7.424999) (end 44.74 8.75) (width 0.8) (layer "B.Cu") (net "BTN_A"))
 (segment (start 61.099999 47.4) (end 62.5 48.8) (width 0.8) (layer "B.Cu") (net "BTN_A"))
 (segment (start 62.5 48.8) (end 62.5 54) (width 0.8) (layer "B.Cu") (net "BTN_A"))
 (segment (start 44.74 13.5) (end 46.24 15) (width 0.8) (layer "B.Cu") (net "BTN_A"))
 (segment (start 59.699999 46) (end 61.099999 47.4) (width 0.8) (layer "B.Cu") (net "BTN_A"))
 (segment (start 44.74 8.75) (end 44.74 13.5) (width 0.8) (layer "B.Cu") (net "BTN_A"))
 (segment (start 59.699999 16.5) (end 59.699999 46) (width 0.8) (layer "B.Cu") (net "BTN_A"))
 (segment (start 46.24 15) (end 58.199999 15) (width 0.8) (layer "B.Cu") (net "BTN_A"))
 (segment (start 59.599999 13.5) (end 61.099999 15) (width 0.8) (layer "B.Cu") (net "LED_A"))
 (segment (start 48.78 13.5) (end 59.599999 13.5) (width 0.8) (layer "B.Cu") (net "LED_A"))
 (segment (start 47.28 8.75) (end 47.28 12) (width 0.8) (layer "B.Cu") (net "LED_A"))
 (segment (start 61.099999 44.5) (end 62.599999 46) (width 0.8) (layer "B.Cu") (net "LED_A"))
 (segment (start 47.28 12) (end 48.78 13.5) (width 0.8) (layer "B.Cu") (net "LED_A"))
 (segment (start 62.599999 46) (end 63.5 46) (width 0.8) (layer "B.Cu") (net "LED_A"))
 (segment (start 61.099999 15) (end 61.099999 44.5) (width 0.8) (layer "B.Cu") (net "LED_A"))
 (segment (start 63.5 46) (end 65 47.5) (width 0.8) (layer "B.Cu") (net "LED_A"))
 (segment (start 65 47.5) (end 65 54) (width 0.8) (layer "B.Cu") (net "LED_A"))
 (segment (start 51.32 12) (end 61 12) (width 0.8) (layer "B.Cu") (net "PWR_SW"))
 (segment (start 67.5 40.5) (end 67.5 43) (width 0.8) (layer "B.Cu") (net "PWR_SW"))
 (segment (start 66 39) (end 67.5 40.5) (width 0.8) (layer "B.Cu") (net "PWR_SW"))
 (segment (start 62.5 37.5) (end 64 39) (width 0.8) (layer "B.Cu") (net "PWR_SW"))
 (segment (start 62.5 13.5) (end 62.5 37.5) (width 0.8) (layer "B.Cu") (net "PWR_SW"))
 (segment (start 49.82 10.5) (end 51.32 12) (width 0.8) (layer "B.Cu") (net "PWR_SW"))
 (segment (start 61 12) (end 62.5 13.5) (width 0.8) (layer "B.Cu") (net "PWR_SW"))
 (segment (start 64 39) (end 66 39) (width 0.8) (layer "B.Cu") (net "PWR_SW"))
 (segment (start 49.82 8.75) (end 49.82 10.5) (width 0.8) (layer "B.Cu") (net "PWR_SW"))
 (segment (start 14.259999 31.25) (end 14.9125 35) (width 1) (layer "B.Cu") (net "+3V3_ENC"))
 (segment (start 14.9125 35) (end 14.95 37.3625) (width 1) (layer "B.Cu") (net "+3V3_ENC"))
 (segment (start 19.34 31.25) (end 19.34 33) (width 1) (layer "B.Cu") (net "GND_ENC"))
 (segment (start 17.5 34.84) (end 17.5 43) (width 1) (layer "B.Cu") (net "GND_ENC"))
 (segment (start 19.34 33) (end 17.5 34.84) (width 1) (layer "B.Cu") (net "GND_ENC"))
 (segment (start 9.899999 35) (end 13.0875 35) (width 0.8) (layer "B.Cu") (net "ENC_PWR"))
 (segment (start 24.42 29.5) (end 22.92 28) (width 0.8) (layer "B.Cu") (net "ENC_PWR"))
 (segment (start 22.92 28) (end 9.899999 28) (width 0.8) (layer "B.Cu") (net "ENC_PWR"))
 (segment (start 24.42 31.25) (end 24.42 29.5) (width 0.8) (layer "B.Cu") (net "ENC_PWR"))
 (segment (start 13.0875 35) (end 13.05 37.3625) (width 0.8) (layer "B.Cu") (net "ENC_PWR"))
 (segment (start 8.399999 29.5) (end 8.399999 33.5) (width 0.8) (layer "B.Cu") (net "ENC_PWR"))
 (segment (start 8.399999 33.5) (end 9.899999 35) (width 0.8) (layer "B.Cu") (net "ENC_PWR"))
 (segment (start 9.899999 28) (end 8.399999 29.5) (width 0.8) (layer "B.Cu") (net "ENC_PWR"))
 (segment (start 26.96 32.625) (end 25.585 34) (width 0.8) (layer "B.Cu") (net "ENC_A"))
 (segment (start 20 35.5) (end 20 45.775) (width 0.8) (layer "B.Cu") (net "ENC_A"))
 (segment (start 26.96 31.25) (end 26.96 32.625) (width 0.8) (layer "B.Cu") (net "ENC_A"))
 (segment (start 25.585 34) (end 21.5 34) (width 0.8) (layer "B.Cu") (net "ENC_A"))
 (segment (start 21.5 34) (end 20 35.5) (width 0.8) (layer "B.Cu") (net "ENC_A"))
 (segment (start 22.5 36.9) (end 22.5 45.775) (width 0.8) (layer "B.Cu") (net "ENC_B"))
 (segment (start 29.5 31.25) (end 29.5 33.9) (width 0.8) (layer "B.Cu") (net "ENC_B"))
 (segment (start 28 35.4) (end 24 35.4) (width 0.8) (layer "B.Cu") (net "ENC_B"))
 (segment (start 24 35.4) (end 22.5 36.9) (width 0.8) (layer "B.Cu") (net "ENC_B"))
 (segment (start 29.5 33.9) (end 28 35.4) (width 0.8) (layer "B.Cu") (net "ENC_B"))
 (segment (start 38.16 45.6) (end 28.5 45.6) (width 0.8) (layer "B.Cu") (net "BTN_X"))
 (segment (start 39.66 44.1) (end 38.16 45.6) (width 0.8) (layer "B.Cu") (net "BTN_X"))
 (segment (start 39.66 31.25) (end 39.66 44.1) (width 0.8) (layer "B.Cu") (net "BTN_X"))
 (segment (start 28.5 45.6) (end 27 47.1) (width 0.8) (layer "B.Cu") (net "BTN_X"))
 (segment (start 27 47.1) (end 27 54) (width 0.8) (layer "B.Cu") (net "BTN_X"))
 (segment (start 31 47) (end 29.5 48.5) (width 0.8) (layer "B.Cu") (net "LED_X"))
 (segment (start 29.5 48.5) (end 29.5 54) (width 0.8) (layer "B.Cu") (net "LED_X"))
 (segment (start 42.2 31.25) (end 42.2 45.5) (width 0.8) (layer "B.Cu") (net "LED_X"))
 (segment (start 40.7 47) (end 31 47) (width 0.8) (layer "B.Cu") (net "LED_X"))
 (segment (start 42.2 45.5) (end 40.7 47) (width 0.8) (layer "B.Cu") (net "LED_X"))
 (segment (start 45.78 48.4) (end 42 48.4) (width 0.8) (layer "B.Cu") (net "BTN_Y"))
 (segment (start 42 48.4) (end 40.5 49.9) (width 0.8) (layer "B.Cu") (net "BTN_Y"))
 (segment (start 47.28 31.25) (end 47.28 46.9) (width 0.8) (layer "B.Cu") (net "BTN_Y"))
 (segment (start 47.28 46.9) (end 45.78 48.4) (width 0.8) (layer "B.Cu") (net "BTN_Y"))
 (segment (start 40.5 49.9) (end 40.5 54) (width 0.8) (layer "B.Cu") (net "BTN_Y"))
 (segment (start 43 51.3) (end 43 54) (width 0.8) (layer "B.Cu") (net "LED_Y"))
 (segment (start 49.82 31.25) (end 49.82 48.3) (width 0.8) (layer "B.Cu") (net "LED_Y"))
 (segment (start 49.82 48.3) (end 48.32 49.8) (width 0.8) (layer "B.Cu") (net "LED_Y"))
 (segment (start 48.32 49.8) (end 44.5 49.8) (width 0.8) (layer "B.Cu") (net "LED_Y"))
 (segment (start 44.5 49.8) (end 43 51.3) (width 0.8) (layer "B.Cu") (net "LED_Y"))
 (segment (start 12.489999 9.7) (end 12.489999 3.7) (width 1) (layer "B.Cu") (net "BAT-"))
 (segment (start 68.5 3.7) (end 68.5 32.25) (width 1) (layer "B.Cu") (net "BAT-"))
 (segment (start 68.5 32.25) (end 67.25 33.5) (width 1) (layer "B.Cu") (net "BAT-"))
 (segment (start 13.989999 2.2) (end 67 2.2) (width 1) (layer "B.Cu") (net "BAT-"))
 (segment (start 67 2.2) (end 68.5 3.7) (width 1) (layer "B.Cu") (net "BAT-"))
 (segment (start 67.25 33.5) (end 66 33.5) (width 1) (layer "B.Cu") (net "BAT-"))
 (segment (start 12.489999 3.7) (end 13.989999 2.2) (width 1) (layer "B.Cu") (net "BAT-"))
 (segment (start 64.5 3.7) (end 66 5.2) (width 1) (layer "B.Cu") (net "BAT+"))
 (segment (start 16.299999 5.2) (end 17.799999 3.7) (width 1) (layer "B.Cu") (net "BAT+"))
 (segment (start 66 5.2) (end 66 31.5) (width 1) (layer "B.Cu") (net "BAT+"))
 (segment (start 16.299999 9.7) (end 16.299999 5.2) (width 1) (layer "B.Cu") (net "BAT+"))
 (segment (start 17.799999 3.7) (end 64.5 3.7) (width 1) (layer "B.Cu") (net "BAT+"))
 (segment (start 14 39.2375) (end 14 46.1) (width 1) (layer "B.Cu") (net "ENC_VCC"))
 (segment (start 14 46.1) (end 15.5 47.6) (width 1) (layer "B.Cu") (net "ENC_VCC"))
 (segment (start 15.5 47.6) (end 23.5 47.6) (width 1) (layer "B.Cu") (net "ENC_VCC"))
 (segment (start 25 46.1) (end 25 43) (width 1) (layer "B.Cu") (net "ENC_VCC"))
 (segment (start 23.5 47.6) (end 25 46.1) (width 1) (layer "B.Cu") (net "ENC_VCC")))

